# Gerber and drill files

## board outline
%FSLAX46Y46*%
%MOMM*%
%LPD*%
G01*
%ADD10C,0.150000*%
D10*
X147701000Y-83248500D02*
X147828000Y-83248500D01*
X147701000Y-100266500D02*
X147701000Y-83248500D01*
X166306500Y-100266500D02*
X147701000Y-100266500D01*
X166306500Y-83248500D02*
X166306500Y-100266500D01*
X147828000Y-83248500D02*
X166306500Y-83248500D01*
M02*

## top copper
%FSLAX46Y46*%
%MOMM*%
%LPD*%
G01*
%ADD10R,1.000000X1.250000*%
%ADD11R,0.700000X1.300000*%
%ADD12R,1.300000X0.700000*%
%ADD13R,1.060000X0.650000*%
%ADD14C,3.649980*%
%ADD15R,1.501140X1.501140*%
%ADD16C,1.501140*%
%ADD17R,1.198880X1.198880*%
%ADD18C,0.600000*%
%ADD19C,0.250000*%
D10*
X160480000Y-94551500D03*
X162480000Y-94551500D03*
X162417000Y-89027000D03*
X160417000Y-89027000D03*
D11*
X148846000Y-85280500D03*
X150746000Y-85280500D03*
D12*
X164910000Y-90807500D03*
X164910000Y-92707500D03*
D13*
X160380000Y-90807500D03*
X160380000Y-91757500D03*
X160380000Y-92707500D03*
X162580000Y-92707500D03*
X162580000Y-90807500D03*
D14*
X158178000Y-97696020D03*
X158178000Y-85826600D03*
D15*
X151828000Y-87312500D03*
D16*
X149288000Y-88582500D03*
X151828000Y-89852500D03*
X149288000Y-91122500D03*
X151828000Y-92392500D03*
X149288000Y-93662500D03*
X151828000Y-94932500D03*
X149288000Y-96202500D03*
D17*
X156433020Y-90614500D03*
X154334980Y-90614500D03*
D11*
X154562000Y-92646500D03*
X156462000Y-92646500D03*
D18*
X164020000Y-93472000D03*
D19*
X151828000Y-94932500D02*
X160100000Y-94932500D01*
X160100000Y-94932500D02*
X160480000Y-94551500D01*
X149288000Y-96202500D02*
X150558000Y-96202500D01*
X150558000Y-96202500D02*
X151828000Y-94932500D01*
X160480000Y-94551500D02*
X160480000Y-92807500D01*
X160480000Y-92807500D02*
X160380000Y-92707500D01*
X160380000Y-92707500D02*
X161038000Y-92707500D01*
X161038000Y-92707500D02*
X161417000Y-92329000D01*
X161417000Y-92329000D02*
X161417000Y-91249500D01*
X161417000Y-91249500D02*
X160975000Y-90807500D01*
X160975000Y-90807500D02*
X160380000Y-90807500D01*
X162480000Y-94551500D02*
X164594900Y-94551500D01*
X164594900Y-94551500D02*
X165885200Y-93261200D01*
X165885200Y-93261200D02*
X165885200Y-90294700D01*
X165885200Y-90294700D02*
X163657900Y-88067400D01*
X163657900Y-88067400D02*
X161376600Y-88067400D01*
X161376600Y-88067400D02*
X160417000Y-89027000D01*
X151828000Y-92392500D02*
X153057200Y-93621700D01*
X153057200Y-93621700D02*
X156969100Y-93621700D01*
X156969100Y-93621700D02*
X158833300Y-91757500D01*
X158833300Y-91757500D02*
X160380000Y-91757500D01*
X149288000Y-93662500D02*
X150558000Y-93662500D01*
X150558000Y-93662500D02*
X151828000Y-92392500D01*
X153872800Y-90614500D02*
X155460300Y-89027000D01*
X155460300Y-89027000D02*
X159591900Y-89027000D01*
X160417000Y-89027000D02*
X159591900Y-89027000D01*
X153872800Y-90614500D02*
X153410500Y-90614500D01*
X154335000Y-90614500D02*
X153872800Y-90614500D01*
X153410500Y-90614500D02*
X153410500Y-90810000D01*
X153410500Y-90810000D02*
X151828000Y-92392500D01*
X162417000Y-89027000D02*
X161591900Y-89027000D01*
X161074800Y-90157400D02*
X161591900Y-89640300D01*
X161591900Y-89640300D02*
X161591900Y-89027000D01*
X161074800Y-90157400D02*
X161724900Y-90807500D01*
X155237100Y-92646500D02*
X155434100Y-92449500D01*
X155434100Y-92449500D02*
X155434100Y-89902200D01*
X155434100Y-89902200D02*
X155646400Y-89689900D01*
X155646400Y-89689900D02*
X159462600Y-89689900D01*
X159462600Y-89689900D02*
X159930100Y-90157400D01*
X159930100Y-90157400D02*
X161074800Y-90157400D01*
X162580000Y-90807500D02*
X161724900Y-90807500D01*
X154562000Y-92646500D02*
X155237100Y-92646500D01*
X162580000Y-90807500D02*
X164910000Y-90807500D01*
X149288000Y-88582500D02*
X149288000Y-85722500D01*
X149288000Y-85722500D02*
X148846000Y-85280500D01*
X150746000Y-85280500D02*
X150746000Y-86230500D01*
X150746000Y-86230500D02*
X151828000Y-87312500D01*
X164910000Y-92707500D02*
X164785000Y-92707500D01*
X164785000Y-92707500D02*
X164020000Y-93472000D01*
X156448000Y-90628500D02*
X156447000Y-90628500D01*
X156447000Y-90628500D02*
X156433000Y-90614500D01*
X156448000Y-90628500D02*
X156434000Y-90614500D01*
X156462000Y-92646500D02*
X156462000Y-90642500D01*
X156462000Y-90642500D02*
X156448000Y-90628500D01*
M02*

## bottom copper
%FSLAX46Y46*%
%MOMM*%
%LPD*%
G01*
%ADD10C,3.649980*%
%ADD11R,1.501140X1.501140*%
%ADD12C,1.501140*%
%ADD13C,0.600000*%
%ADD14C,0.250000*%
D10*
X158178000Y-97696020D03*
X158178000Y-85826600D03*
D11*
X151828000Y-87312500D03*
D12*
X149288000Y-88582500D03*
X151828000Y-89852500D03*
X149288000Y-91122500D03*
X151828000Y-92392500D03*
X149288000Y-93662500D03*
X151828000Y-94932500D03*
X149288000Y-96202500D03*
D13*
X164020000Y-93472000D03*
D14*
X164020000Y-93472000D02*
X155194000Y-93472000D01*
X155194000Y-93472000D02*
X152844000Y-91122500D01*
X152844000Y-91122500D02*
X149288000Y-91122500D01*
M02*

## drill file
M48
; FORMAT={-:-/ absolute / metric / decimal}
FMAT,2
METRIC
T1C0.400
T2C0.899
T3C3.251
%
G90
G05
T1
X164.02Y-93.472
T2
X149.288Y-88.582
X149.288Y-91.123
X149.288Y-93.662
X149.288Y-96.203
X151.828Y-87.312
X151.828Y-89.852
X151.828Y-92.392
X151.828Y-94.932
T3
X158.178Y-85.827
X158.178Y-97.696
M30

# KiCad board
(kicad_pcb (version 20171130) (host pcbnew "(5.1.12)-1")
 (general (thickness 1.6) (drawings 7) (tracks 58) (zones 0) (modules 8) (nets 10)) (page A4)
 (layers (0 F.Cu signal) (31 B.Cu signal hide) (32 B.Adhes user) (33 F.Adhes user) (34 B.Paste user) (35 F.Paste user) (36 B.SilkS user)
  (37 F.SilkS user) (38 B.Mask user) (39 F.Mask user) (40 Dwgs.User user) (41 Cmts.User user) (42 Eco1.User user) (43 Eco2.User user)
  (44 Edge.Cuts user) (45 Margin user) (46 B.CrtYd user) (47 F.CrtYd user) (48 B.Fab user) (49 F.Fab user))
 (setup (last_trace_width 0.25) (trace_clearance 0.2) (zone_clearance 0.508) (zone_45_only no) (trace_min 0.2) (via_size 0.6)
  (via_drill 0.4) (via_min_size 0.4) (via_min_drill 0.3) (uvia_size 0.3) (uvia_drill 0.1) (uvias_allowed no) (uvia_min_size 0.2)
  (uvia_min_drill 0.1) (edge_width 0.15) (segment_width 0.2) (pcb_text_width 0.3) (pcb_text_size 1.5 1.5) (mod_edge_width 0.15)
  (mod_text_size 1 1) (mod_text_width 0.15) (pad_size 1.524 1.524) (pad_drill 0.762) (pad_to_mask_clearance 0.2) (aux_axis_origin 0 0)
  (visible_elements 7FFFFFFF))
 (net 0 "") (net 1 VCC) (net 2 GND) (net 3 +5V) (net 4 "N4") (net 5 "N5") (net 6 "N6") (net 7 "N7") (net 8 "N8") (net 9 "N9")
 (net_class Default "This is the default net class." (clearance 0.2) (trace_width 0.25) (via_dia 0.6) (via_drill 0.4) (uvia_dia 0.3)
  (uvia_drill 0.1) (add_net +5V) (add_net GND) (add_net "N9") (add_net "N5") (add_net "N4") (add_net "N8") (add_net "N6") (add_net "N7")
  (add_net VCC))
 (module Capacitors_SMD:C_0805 (layer F.Cu) (at 161.48 94.5515)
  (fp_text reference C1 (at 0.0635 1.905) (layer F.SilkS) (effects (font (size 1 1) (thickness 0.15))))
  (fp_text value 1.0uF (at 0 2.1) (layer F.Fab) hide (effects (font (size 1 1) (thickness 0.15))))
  (pad 1 smd rect (at -1 0) (size 1 1.25) (layers F.Cu F.Paste F.Mask) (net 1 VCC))
  (pad 2 smd rect (at 1 0) (size 1 1.25) (layers F.Cu F.Paste F.Mask) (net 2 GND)))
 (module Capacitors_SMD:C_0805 (layer F.Cu) (at 161.417 89.027 180)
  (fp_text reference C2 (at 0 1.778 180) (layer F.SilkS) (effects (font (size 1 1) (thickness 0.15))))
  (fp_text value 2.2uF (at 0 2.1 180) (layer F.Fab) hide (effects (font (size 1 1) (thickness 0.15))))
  (pad 1 smd rect (at -1 0 180) (size 1 1.25) (layers F.Cu F.Paste F.Mask) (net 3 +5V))
  (pad 2 smd rect (at 1 0 180) (size 1 1.25) (layers F.Cu F.Paste F.Mask) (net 2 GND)))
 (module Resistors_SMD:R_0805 (layer F.Cu) (at 149.796 85.2805)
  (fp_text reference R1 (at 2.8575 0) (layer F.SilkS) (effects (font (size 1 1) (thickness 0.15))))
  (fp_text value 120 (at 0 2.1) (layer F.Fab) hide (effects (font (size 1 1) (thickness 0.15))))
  (pad 1 smd rect (at -0.95 0) (size 0.7 1.3) (layers F.Cu F.Paste F.Mask) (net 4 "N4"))
  (pad 2 smd rect (at 0.95 0) (size 0.7 1.3) (layers F.Cu F.Paste F.Mask) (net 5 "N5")))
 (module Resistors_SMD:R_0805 (layer F.Cu) (at 164.91 91.7575 270)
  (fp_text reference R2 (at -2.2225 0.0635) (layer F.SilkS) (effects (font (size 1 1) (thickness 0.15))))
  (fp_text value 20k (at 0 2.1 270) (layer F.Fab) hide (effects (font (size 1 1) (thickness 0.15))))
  (pad 1 smd rect (at -0.95 0 270) (size 0.7 1.3) (layers F.Cu F.Paste F.Mask) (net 3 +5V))
  (pad 2 smd rect (at 0.95 0 270) (size 0.7 1.3) (layers F.Cu F.Paste F.Mask) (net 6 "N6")))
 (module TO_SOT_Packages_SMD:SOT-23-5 (layer F.Cu) (at 161.48 91.7575)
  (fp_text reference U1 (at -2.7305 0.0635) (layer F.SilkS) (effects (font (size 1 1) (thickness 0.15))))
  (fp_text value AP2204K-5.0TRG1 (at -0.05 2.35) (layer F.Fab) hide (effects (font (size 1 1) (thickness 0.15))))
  (pad 1 smd rect (at -1.1 -0.95) (size 1.06 0.65) (layers F.Cu F.Paste F.Mask) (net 1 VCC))
  (pad 2 smd rect (at -1.1 0) (size 1.06 0.65) (layers F.Cu F.Paste F.Mask) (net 2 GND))
  (pad 3 smd rect (at -1.1 0.95) (size 1.06 0.65) (layers F.Cu F.Paste F.Mask) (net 1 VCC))
  (pad 4 smd rect (at 1.1 0.95) (size 1.06 0.65) (layers F.Cu F.Paste F.Mask) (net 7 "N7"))
  (pad 5 smd rect (at 1.1 -0.95) (size 1.06 0.65) (layers F.Cu F.Paste F.Mask) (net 3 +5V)))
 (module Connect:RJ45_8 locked (layer B.Cu) (at 158.178 91.7575 270)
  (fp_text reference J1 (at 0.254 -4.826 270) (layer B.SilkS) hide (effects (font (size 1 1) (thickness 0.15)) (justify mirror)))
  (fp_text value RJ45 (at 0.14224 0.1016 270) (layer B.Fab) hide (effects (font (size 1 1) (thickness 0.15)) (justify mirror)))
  (pad Hole np_thru_hole circle (at 5.93852 0 270) (size 3.64998 3.64998) (drill 3.2512) (layers *.Cu *.SilkS *.Mask))
  (pad Hole np_thru_hole circle (at -5.9309 0 270) (size 3.64998 3.64998) (drill 3.2512) (layers *.Cu *.SilkS *.Mask))
  (pad 1 thru_hole rect (at -4.445 6.35 270) (size 1.50114 1.50114) (drill 0.89916) (layers *.Cu *.Mask B.SilkS) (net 5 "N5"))
  (pad 2 thru_hole circle (at -3.175 8.89 270) (size 1.50114 1.50114) (drill 0.89916) (layers *.Cu *.Mask B.SilkS) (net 4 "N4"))
  (pad 3 thru_hole circle (at -1.905 6.35 270) (size 1.50114 1.50114) (drill 0.89916) (layers *.Cu *.Mask B.SilkS) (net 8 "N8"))
  (pad 4 thru_hole circle (at -0.635 8.89 270) (size 1.50114 1.50114) (drill 0.89916) (layers *.Cu *.Mask B.SilkS) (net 6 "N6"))
  (pad 5 thru_hole circle (at 0.635 6.35 270) (size 1.50114 1.50114) (drill 0.89916) (layers *.Cu *.Mask B.SilkS) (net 2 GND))
  (pad 6 thru_hole circle (at 1.905 8.89 270) (size 1.50114 1.50114) (drill 0.89916) (layers *.Cu *.Mask B.SilkS) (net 2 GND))
  (pad 7 thru_hole circle (at 3.175 6.35 270) (size 1.50114 1.50114) (drill 0.89916) (layers *.Cu *.Mask B.SilkS) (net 1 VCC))
  (pad 8 thru_hole circle (at 4.445 8.89 270) (size 1.50114 1.50114) (drill 0.89916) (layers *.Cu *.Mask B.SilkS) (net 1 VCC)))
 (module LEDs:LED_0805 (layer F.Cu) (at 155.384 90.6145)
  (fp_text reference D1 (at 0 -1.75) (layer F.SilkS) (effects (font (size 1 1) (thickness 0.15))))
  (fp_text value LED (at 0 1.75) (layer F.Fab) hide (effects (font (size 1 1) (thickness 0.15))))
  (pad 2 smd rect (at 1.04902 0 180) (size 1.19888 1.19888) (layers F.Cu F.Paste F.Mask) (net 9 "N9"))
  (pad 1 smd rect (at -1.04902 0 180) (size 1.19888 1.19888) (layers F.Cu F.Paste F.Mask) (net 2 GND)))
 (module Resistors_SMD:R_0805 (layer F.Cu) (at 155.512 92.6465)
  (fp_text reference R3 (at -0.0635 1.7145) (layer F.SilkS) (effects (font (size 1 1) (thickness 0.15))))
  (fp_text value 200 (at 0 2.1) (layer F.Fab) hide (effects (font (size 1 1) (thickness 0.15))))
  (pad 1 smd rect (at -0.95 0) (size 0.7 1.3) (layers F.Cu F.Paste F.Mask) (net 3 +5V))
  (pad 2 smd rect (at 0.95 0) (size 0.7 1.3) (layers F.Cu F.Paste F.Mask) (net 9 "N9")))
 (gr_line (start 147.701 83.2485) (end 147.828 83.2485) (angle 90) (layer Edge.Cuts) (width 0.15))
 (gr_line (start 147.701 100.2665) (end 147.701 83.2485) (angle 90) (layer Edge.Cuts) (width 0.15))
 (gr_line (start 166.3065 100.2665) (end 147.701 100.2665) (angle 90) (layer Edge.Cuts) (width 0.15))
 (gr_line (start 166.3065 83.2485) (end 166.3065 100.2665) (angle 90) (layer Edge.Cuts) (width 0.15))
 (gr_line (start 147.828 83.2485) (end 166.3065 83.2485) (angle 90) (layer Edge.Cuts) (width 0.15))
 (segment (start 151.828 94.9325) (end 160.1 94.9325) (width 0.25) (layer F.Cu) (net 1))
 (segment (start 160.1 94.9325) (end 160.48 94.5515) (width 0.25) (layer F.Cu) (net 1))
 (segment (start 149.288 96.2025) (end 150.558 96.2025) (width 0.25) (layer F.Cu) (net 1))
 (segment (start 150.558 96.2025) (end 151.828 94.9325) (width 0.25) (layer F.Cu) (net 1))
 (segment (start 160.48 94.5515) (end 160.48 92.8075) (width 0.25) (layer F.Cu) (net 1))
 (segment (start 160.48 92.8075) (end 160.38 92.7075) (width 0.25) (layer F.Cu) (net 1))
 (segment (start 160.38 92.7075) (end 161.038 92.7075) (width 0.25) (layer F.Cu) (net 1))
 (segment (start 161.038 92.7075) (end 161.417 92.329) (width 0.25) (layer F.Cu) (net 1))
 (segment (start 161.417 92.329) (end 161.417 91.2495) (width 0.25) (layer F.Cu) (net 1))
 (segment (start 161.417 91.2495) (end 160.975 90.8075) (width 0.25) (layer F.Cu) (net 1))
 (segment (start 160.975 90.8075) (end 160.38 90.8075) (width 0.25) (layer F.Cu) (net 1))
 (segment (start 162.48 94.5515) (end 164.5949 94.5515) (width 0.25) (layer F.Cu) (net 2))
 (segment (start 164.5949 94.5515) (end 165.8852 93.2612) (width 0.25) (layer F.Cu) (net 2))
 (segment (start 165.8852 93.2612) (end 165.8852 90.2947) (width 0.25) (layer F.Cu) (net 2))
 (segment (start 165.8852 90.2947) (end 163.6579 88.0674) (width 0.25) (layer F.Cu) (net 2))
 (segment (start 163.6579 88.0674) (end 161.3766 88.0674) (width 0.25) (layer F.Cu) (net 2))
 (segment (start 161.3766 88.0674) (end 160.417 89.027) (width 0.25) (layer F.Cu) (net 2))
 (segment (start 151.828 92.3925) (end 153.0572 93.6217) (width 0.25) (layer F.Cu) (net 2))
 (segment (start 153.0572 93.6217) (end 156.9691 93.6217) (width 0.25) (layer F.Cu) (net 2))
 (segment (start 156.9691 93.6217) (end 158.8333 91.7575) (width 0.25) (layer F.Cu) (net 2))
 (segment (start 158.8333 91.7575) (end 160.38 91.7575) (width 0.25) (layer F.Cu) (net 2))
 (segment (start 149.288 93.6625) (end 150.558 93.6625) (width 0.25) (layer F.Cu) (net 2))
 (segment (start 150.558 93.6625) (end 151.828 92.3925) (width 0.25) (layer F.Cu) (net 2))
 (segment (start 153.8728 90.6145) (end 155.4603 89.027) (width 0.25) (layer F.Cu) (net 2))
 (segment (start 155.4603 89.027) (end 159.5919 89.027) (width 0.25) (layer F.Cu) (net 2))
 (segment (start 160.417 89.027) (end 159.5919 89.027) (width 0.25) (layer F.Cu) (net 2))
 (segment (start 153.8728 90.6145) (end 153.4105 90.6145) (width 0.25) (layer F.Cu) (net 2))
 (segment (start 154.335 90.6145) (end 153.8728 90.6145) (width 0.25) (layer F.Cu) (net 2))
 (segment (start 153.4105 90.6145) (end 153.4105 90.81) (width 0.25) (layer F.Cu) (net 2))
 (segment (start 153.4105 90.81) (end 151.828 92.3925) (width 0.25) (layer F.Cu) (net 2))
 (segment (start 162.417 89.027) (end 161.5919 89.027) (width 0.25) (layer F.Cu) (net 3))
 (segment (start 161.0748 90.1574) (end 161.5919 89.6403) (width 0.25) (layer F.Cu) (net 3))
 (segment (start 161.5919 89.6403) (end 161.5919 89.027) (width 0.25) (layer F.Cu) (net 3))
 (segment (start 161.0748 90.1574) (end 161.7249 90.8075) (width 0.25) (layer F.Cu) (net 3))
 (segment (start 155.2371 92.6465) (end 155.4341 92.4495) (width 0.25) (layer F.Cu) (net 3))
 (segment (start 155.4341 92.4495) (end 155.4341 89.9022) (width 0.25) (layer F.Cu) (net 3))
 (segment (start 155.4341 89.9022) (end 155.6464 89.6899) (width 0.25) (layer F.Cu) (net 3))
 (segment (start 155.6464 89.6899) (end 159.4626 89.6899) (width 0.25) (layer F.Cu) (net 3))
 (segment (start 159.4626 89.6899) (end 159.9301 90.1574) (width 0.25) (layer F.Cu) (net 3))
 (segment (start 159.9301 90.1574) (end 161.0748 90.1574) (width 0.25) (layer F.Cu) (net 3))
 (segment (start 162.58 90.8075) (end 161.7249 90.8075) (width 0.25) (layer F.Cu) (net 3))
 (segment (start 154.562 92.6465) (end 155.2371 92.6465) (width 0.25) (layer F.Cu) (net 3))
 (segment (start 162.58 90.8075) (end 164.91 90.8075) (width 0.25) (layer F.Cu) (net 3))
 (segment (start 149.288 88.5825) (end 149.288 85.7225) (width 0.25) (layer F.Cu) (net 4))
 (segment (start 149.288 85.7225) (end 148.846 85.2805) (width 0.25) (layer F.Cu) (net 4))
 (segment (start 150.746 85.2805) (end 150.746 86.2305) (width 0.25) (layer F.Cu) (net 5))
 (segment (start 150.746 86.2305) (end 151.828 87.3125) (width 0.25) (layer F.Cu) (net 5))
 (segment (start 164.91 92.7075) (end 164.785 92.7075) (width 0.25) (layer F.Cu) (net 6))
 (segment (start 164.785 92.7075) (end 164.02 93.472) (width 0.25) (layer F.Cu) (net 6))
 (segment (start 164.02 93.472) (end 155.194 93.472) (width 0.25) (layer B.Cu) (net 6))
 (segment (start 155.194 93.472) (end 152.844 91.1225) (width 0.25) (layer B.Cu) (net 6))
 (segment (start 152.844 91.1225) (end 149.288 91.1225) (width 0.25) (layer B.Cu) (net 6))
 (via (at 164.02 93.472) (size 0.6) (layers F.Cu B.Cu) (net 6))
 (segment (start 156.448 90.6285) (end 156.447 90.6285) (width 0.25) (layer F.Cu) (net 9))
 (segment (start 156.447 90.6285) (end 156.433 90.6145) (width 0.25) (layer F.Cu) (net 9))
 (segment (start 156.448 90.6285) (end 156.434 90.6145) (width 0.25) (layer F.Cu) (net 9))
 (segment (start 156.462 92.6465) (end 156.462 90.6425) (width 0.25) (layer F.Cu) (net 9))
 (segment (start 156.462 90.6425) (end 156.448 90.6285) (width 0.25) (layer F.Cu) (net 9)))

